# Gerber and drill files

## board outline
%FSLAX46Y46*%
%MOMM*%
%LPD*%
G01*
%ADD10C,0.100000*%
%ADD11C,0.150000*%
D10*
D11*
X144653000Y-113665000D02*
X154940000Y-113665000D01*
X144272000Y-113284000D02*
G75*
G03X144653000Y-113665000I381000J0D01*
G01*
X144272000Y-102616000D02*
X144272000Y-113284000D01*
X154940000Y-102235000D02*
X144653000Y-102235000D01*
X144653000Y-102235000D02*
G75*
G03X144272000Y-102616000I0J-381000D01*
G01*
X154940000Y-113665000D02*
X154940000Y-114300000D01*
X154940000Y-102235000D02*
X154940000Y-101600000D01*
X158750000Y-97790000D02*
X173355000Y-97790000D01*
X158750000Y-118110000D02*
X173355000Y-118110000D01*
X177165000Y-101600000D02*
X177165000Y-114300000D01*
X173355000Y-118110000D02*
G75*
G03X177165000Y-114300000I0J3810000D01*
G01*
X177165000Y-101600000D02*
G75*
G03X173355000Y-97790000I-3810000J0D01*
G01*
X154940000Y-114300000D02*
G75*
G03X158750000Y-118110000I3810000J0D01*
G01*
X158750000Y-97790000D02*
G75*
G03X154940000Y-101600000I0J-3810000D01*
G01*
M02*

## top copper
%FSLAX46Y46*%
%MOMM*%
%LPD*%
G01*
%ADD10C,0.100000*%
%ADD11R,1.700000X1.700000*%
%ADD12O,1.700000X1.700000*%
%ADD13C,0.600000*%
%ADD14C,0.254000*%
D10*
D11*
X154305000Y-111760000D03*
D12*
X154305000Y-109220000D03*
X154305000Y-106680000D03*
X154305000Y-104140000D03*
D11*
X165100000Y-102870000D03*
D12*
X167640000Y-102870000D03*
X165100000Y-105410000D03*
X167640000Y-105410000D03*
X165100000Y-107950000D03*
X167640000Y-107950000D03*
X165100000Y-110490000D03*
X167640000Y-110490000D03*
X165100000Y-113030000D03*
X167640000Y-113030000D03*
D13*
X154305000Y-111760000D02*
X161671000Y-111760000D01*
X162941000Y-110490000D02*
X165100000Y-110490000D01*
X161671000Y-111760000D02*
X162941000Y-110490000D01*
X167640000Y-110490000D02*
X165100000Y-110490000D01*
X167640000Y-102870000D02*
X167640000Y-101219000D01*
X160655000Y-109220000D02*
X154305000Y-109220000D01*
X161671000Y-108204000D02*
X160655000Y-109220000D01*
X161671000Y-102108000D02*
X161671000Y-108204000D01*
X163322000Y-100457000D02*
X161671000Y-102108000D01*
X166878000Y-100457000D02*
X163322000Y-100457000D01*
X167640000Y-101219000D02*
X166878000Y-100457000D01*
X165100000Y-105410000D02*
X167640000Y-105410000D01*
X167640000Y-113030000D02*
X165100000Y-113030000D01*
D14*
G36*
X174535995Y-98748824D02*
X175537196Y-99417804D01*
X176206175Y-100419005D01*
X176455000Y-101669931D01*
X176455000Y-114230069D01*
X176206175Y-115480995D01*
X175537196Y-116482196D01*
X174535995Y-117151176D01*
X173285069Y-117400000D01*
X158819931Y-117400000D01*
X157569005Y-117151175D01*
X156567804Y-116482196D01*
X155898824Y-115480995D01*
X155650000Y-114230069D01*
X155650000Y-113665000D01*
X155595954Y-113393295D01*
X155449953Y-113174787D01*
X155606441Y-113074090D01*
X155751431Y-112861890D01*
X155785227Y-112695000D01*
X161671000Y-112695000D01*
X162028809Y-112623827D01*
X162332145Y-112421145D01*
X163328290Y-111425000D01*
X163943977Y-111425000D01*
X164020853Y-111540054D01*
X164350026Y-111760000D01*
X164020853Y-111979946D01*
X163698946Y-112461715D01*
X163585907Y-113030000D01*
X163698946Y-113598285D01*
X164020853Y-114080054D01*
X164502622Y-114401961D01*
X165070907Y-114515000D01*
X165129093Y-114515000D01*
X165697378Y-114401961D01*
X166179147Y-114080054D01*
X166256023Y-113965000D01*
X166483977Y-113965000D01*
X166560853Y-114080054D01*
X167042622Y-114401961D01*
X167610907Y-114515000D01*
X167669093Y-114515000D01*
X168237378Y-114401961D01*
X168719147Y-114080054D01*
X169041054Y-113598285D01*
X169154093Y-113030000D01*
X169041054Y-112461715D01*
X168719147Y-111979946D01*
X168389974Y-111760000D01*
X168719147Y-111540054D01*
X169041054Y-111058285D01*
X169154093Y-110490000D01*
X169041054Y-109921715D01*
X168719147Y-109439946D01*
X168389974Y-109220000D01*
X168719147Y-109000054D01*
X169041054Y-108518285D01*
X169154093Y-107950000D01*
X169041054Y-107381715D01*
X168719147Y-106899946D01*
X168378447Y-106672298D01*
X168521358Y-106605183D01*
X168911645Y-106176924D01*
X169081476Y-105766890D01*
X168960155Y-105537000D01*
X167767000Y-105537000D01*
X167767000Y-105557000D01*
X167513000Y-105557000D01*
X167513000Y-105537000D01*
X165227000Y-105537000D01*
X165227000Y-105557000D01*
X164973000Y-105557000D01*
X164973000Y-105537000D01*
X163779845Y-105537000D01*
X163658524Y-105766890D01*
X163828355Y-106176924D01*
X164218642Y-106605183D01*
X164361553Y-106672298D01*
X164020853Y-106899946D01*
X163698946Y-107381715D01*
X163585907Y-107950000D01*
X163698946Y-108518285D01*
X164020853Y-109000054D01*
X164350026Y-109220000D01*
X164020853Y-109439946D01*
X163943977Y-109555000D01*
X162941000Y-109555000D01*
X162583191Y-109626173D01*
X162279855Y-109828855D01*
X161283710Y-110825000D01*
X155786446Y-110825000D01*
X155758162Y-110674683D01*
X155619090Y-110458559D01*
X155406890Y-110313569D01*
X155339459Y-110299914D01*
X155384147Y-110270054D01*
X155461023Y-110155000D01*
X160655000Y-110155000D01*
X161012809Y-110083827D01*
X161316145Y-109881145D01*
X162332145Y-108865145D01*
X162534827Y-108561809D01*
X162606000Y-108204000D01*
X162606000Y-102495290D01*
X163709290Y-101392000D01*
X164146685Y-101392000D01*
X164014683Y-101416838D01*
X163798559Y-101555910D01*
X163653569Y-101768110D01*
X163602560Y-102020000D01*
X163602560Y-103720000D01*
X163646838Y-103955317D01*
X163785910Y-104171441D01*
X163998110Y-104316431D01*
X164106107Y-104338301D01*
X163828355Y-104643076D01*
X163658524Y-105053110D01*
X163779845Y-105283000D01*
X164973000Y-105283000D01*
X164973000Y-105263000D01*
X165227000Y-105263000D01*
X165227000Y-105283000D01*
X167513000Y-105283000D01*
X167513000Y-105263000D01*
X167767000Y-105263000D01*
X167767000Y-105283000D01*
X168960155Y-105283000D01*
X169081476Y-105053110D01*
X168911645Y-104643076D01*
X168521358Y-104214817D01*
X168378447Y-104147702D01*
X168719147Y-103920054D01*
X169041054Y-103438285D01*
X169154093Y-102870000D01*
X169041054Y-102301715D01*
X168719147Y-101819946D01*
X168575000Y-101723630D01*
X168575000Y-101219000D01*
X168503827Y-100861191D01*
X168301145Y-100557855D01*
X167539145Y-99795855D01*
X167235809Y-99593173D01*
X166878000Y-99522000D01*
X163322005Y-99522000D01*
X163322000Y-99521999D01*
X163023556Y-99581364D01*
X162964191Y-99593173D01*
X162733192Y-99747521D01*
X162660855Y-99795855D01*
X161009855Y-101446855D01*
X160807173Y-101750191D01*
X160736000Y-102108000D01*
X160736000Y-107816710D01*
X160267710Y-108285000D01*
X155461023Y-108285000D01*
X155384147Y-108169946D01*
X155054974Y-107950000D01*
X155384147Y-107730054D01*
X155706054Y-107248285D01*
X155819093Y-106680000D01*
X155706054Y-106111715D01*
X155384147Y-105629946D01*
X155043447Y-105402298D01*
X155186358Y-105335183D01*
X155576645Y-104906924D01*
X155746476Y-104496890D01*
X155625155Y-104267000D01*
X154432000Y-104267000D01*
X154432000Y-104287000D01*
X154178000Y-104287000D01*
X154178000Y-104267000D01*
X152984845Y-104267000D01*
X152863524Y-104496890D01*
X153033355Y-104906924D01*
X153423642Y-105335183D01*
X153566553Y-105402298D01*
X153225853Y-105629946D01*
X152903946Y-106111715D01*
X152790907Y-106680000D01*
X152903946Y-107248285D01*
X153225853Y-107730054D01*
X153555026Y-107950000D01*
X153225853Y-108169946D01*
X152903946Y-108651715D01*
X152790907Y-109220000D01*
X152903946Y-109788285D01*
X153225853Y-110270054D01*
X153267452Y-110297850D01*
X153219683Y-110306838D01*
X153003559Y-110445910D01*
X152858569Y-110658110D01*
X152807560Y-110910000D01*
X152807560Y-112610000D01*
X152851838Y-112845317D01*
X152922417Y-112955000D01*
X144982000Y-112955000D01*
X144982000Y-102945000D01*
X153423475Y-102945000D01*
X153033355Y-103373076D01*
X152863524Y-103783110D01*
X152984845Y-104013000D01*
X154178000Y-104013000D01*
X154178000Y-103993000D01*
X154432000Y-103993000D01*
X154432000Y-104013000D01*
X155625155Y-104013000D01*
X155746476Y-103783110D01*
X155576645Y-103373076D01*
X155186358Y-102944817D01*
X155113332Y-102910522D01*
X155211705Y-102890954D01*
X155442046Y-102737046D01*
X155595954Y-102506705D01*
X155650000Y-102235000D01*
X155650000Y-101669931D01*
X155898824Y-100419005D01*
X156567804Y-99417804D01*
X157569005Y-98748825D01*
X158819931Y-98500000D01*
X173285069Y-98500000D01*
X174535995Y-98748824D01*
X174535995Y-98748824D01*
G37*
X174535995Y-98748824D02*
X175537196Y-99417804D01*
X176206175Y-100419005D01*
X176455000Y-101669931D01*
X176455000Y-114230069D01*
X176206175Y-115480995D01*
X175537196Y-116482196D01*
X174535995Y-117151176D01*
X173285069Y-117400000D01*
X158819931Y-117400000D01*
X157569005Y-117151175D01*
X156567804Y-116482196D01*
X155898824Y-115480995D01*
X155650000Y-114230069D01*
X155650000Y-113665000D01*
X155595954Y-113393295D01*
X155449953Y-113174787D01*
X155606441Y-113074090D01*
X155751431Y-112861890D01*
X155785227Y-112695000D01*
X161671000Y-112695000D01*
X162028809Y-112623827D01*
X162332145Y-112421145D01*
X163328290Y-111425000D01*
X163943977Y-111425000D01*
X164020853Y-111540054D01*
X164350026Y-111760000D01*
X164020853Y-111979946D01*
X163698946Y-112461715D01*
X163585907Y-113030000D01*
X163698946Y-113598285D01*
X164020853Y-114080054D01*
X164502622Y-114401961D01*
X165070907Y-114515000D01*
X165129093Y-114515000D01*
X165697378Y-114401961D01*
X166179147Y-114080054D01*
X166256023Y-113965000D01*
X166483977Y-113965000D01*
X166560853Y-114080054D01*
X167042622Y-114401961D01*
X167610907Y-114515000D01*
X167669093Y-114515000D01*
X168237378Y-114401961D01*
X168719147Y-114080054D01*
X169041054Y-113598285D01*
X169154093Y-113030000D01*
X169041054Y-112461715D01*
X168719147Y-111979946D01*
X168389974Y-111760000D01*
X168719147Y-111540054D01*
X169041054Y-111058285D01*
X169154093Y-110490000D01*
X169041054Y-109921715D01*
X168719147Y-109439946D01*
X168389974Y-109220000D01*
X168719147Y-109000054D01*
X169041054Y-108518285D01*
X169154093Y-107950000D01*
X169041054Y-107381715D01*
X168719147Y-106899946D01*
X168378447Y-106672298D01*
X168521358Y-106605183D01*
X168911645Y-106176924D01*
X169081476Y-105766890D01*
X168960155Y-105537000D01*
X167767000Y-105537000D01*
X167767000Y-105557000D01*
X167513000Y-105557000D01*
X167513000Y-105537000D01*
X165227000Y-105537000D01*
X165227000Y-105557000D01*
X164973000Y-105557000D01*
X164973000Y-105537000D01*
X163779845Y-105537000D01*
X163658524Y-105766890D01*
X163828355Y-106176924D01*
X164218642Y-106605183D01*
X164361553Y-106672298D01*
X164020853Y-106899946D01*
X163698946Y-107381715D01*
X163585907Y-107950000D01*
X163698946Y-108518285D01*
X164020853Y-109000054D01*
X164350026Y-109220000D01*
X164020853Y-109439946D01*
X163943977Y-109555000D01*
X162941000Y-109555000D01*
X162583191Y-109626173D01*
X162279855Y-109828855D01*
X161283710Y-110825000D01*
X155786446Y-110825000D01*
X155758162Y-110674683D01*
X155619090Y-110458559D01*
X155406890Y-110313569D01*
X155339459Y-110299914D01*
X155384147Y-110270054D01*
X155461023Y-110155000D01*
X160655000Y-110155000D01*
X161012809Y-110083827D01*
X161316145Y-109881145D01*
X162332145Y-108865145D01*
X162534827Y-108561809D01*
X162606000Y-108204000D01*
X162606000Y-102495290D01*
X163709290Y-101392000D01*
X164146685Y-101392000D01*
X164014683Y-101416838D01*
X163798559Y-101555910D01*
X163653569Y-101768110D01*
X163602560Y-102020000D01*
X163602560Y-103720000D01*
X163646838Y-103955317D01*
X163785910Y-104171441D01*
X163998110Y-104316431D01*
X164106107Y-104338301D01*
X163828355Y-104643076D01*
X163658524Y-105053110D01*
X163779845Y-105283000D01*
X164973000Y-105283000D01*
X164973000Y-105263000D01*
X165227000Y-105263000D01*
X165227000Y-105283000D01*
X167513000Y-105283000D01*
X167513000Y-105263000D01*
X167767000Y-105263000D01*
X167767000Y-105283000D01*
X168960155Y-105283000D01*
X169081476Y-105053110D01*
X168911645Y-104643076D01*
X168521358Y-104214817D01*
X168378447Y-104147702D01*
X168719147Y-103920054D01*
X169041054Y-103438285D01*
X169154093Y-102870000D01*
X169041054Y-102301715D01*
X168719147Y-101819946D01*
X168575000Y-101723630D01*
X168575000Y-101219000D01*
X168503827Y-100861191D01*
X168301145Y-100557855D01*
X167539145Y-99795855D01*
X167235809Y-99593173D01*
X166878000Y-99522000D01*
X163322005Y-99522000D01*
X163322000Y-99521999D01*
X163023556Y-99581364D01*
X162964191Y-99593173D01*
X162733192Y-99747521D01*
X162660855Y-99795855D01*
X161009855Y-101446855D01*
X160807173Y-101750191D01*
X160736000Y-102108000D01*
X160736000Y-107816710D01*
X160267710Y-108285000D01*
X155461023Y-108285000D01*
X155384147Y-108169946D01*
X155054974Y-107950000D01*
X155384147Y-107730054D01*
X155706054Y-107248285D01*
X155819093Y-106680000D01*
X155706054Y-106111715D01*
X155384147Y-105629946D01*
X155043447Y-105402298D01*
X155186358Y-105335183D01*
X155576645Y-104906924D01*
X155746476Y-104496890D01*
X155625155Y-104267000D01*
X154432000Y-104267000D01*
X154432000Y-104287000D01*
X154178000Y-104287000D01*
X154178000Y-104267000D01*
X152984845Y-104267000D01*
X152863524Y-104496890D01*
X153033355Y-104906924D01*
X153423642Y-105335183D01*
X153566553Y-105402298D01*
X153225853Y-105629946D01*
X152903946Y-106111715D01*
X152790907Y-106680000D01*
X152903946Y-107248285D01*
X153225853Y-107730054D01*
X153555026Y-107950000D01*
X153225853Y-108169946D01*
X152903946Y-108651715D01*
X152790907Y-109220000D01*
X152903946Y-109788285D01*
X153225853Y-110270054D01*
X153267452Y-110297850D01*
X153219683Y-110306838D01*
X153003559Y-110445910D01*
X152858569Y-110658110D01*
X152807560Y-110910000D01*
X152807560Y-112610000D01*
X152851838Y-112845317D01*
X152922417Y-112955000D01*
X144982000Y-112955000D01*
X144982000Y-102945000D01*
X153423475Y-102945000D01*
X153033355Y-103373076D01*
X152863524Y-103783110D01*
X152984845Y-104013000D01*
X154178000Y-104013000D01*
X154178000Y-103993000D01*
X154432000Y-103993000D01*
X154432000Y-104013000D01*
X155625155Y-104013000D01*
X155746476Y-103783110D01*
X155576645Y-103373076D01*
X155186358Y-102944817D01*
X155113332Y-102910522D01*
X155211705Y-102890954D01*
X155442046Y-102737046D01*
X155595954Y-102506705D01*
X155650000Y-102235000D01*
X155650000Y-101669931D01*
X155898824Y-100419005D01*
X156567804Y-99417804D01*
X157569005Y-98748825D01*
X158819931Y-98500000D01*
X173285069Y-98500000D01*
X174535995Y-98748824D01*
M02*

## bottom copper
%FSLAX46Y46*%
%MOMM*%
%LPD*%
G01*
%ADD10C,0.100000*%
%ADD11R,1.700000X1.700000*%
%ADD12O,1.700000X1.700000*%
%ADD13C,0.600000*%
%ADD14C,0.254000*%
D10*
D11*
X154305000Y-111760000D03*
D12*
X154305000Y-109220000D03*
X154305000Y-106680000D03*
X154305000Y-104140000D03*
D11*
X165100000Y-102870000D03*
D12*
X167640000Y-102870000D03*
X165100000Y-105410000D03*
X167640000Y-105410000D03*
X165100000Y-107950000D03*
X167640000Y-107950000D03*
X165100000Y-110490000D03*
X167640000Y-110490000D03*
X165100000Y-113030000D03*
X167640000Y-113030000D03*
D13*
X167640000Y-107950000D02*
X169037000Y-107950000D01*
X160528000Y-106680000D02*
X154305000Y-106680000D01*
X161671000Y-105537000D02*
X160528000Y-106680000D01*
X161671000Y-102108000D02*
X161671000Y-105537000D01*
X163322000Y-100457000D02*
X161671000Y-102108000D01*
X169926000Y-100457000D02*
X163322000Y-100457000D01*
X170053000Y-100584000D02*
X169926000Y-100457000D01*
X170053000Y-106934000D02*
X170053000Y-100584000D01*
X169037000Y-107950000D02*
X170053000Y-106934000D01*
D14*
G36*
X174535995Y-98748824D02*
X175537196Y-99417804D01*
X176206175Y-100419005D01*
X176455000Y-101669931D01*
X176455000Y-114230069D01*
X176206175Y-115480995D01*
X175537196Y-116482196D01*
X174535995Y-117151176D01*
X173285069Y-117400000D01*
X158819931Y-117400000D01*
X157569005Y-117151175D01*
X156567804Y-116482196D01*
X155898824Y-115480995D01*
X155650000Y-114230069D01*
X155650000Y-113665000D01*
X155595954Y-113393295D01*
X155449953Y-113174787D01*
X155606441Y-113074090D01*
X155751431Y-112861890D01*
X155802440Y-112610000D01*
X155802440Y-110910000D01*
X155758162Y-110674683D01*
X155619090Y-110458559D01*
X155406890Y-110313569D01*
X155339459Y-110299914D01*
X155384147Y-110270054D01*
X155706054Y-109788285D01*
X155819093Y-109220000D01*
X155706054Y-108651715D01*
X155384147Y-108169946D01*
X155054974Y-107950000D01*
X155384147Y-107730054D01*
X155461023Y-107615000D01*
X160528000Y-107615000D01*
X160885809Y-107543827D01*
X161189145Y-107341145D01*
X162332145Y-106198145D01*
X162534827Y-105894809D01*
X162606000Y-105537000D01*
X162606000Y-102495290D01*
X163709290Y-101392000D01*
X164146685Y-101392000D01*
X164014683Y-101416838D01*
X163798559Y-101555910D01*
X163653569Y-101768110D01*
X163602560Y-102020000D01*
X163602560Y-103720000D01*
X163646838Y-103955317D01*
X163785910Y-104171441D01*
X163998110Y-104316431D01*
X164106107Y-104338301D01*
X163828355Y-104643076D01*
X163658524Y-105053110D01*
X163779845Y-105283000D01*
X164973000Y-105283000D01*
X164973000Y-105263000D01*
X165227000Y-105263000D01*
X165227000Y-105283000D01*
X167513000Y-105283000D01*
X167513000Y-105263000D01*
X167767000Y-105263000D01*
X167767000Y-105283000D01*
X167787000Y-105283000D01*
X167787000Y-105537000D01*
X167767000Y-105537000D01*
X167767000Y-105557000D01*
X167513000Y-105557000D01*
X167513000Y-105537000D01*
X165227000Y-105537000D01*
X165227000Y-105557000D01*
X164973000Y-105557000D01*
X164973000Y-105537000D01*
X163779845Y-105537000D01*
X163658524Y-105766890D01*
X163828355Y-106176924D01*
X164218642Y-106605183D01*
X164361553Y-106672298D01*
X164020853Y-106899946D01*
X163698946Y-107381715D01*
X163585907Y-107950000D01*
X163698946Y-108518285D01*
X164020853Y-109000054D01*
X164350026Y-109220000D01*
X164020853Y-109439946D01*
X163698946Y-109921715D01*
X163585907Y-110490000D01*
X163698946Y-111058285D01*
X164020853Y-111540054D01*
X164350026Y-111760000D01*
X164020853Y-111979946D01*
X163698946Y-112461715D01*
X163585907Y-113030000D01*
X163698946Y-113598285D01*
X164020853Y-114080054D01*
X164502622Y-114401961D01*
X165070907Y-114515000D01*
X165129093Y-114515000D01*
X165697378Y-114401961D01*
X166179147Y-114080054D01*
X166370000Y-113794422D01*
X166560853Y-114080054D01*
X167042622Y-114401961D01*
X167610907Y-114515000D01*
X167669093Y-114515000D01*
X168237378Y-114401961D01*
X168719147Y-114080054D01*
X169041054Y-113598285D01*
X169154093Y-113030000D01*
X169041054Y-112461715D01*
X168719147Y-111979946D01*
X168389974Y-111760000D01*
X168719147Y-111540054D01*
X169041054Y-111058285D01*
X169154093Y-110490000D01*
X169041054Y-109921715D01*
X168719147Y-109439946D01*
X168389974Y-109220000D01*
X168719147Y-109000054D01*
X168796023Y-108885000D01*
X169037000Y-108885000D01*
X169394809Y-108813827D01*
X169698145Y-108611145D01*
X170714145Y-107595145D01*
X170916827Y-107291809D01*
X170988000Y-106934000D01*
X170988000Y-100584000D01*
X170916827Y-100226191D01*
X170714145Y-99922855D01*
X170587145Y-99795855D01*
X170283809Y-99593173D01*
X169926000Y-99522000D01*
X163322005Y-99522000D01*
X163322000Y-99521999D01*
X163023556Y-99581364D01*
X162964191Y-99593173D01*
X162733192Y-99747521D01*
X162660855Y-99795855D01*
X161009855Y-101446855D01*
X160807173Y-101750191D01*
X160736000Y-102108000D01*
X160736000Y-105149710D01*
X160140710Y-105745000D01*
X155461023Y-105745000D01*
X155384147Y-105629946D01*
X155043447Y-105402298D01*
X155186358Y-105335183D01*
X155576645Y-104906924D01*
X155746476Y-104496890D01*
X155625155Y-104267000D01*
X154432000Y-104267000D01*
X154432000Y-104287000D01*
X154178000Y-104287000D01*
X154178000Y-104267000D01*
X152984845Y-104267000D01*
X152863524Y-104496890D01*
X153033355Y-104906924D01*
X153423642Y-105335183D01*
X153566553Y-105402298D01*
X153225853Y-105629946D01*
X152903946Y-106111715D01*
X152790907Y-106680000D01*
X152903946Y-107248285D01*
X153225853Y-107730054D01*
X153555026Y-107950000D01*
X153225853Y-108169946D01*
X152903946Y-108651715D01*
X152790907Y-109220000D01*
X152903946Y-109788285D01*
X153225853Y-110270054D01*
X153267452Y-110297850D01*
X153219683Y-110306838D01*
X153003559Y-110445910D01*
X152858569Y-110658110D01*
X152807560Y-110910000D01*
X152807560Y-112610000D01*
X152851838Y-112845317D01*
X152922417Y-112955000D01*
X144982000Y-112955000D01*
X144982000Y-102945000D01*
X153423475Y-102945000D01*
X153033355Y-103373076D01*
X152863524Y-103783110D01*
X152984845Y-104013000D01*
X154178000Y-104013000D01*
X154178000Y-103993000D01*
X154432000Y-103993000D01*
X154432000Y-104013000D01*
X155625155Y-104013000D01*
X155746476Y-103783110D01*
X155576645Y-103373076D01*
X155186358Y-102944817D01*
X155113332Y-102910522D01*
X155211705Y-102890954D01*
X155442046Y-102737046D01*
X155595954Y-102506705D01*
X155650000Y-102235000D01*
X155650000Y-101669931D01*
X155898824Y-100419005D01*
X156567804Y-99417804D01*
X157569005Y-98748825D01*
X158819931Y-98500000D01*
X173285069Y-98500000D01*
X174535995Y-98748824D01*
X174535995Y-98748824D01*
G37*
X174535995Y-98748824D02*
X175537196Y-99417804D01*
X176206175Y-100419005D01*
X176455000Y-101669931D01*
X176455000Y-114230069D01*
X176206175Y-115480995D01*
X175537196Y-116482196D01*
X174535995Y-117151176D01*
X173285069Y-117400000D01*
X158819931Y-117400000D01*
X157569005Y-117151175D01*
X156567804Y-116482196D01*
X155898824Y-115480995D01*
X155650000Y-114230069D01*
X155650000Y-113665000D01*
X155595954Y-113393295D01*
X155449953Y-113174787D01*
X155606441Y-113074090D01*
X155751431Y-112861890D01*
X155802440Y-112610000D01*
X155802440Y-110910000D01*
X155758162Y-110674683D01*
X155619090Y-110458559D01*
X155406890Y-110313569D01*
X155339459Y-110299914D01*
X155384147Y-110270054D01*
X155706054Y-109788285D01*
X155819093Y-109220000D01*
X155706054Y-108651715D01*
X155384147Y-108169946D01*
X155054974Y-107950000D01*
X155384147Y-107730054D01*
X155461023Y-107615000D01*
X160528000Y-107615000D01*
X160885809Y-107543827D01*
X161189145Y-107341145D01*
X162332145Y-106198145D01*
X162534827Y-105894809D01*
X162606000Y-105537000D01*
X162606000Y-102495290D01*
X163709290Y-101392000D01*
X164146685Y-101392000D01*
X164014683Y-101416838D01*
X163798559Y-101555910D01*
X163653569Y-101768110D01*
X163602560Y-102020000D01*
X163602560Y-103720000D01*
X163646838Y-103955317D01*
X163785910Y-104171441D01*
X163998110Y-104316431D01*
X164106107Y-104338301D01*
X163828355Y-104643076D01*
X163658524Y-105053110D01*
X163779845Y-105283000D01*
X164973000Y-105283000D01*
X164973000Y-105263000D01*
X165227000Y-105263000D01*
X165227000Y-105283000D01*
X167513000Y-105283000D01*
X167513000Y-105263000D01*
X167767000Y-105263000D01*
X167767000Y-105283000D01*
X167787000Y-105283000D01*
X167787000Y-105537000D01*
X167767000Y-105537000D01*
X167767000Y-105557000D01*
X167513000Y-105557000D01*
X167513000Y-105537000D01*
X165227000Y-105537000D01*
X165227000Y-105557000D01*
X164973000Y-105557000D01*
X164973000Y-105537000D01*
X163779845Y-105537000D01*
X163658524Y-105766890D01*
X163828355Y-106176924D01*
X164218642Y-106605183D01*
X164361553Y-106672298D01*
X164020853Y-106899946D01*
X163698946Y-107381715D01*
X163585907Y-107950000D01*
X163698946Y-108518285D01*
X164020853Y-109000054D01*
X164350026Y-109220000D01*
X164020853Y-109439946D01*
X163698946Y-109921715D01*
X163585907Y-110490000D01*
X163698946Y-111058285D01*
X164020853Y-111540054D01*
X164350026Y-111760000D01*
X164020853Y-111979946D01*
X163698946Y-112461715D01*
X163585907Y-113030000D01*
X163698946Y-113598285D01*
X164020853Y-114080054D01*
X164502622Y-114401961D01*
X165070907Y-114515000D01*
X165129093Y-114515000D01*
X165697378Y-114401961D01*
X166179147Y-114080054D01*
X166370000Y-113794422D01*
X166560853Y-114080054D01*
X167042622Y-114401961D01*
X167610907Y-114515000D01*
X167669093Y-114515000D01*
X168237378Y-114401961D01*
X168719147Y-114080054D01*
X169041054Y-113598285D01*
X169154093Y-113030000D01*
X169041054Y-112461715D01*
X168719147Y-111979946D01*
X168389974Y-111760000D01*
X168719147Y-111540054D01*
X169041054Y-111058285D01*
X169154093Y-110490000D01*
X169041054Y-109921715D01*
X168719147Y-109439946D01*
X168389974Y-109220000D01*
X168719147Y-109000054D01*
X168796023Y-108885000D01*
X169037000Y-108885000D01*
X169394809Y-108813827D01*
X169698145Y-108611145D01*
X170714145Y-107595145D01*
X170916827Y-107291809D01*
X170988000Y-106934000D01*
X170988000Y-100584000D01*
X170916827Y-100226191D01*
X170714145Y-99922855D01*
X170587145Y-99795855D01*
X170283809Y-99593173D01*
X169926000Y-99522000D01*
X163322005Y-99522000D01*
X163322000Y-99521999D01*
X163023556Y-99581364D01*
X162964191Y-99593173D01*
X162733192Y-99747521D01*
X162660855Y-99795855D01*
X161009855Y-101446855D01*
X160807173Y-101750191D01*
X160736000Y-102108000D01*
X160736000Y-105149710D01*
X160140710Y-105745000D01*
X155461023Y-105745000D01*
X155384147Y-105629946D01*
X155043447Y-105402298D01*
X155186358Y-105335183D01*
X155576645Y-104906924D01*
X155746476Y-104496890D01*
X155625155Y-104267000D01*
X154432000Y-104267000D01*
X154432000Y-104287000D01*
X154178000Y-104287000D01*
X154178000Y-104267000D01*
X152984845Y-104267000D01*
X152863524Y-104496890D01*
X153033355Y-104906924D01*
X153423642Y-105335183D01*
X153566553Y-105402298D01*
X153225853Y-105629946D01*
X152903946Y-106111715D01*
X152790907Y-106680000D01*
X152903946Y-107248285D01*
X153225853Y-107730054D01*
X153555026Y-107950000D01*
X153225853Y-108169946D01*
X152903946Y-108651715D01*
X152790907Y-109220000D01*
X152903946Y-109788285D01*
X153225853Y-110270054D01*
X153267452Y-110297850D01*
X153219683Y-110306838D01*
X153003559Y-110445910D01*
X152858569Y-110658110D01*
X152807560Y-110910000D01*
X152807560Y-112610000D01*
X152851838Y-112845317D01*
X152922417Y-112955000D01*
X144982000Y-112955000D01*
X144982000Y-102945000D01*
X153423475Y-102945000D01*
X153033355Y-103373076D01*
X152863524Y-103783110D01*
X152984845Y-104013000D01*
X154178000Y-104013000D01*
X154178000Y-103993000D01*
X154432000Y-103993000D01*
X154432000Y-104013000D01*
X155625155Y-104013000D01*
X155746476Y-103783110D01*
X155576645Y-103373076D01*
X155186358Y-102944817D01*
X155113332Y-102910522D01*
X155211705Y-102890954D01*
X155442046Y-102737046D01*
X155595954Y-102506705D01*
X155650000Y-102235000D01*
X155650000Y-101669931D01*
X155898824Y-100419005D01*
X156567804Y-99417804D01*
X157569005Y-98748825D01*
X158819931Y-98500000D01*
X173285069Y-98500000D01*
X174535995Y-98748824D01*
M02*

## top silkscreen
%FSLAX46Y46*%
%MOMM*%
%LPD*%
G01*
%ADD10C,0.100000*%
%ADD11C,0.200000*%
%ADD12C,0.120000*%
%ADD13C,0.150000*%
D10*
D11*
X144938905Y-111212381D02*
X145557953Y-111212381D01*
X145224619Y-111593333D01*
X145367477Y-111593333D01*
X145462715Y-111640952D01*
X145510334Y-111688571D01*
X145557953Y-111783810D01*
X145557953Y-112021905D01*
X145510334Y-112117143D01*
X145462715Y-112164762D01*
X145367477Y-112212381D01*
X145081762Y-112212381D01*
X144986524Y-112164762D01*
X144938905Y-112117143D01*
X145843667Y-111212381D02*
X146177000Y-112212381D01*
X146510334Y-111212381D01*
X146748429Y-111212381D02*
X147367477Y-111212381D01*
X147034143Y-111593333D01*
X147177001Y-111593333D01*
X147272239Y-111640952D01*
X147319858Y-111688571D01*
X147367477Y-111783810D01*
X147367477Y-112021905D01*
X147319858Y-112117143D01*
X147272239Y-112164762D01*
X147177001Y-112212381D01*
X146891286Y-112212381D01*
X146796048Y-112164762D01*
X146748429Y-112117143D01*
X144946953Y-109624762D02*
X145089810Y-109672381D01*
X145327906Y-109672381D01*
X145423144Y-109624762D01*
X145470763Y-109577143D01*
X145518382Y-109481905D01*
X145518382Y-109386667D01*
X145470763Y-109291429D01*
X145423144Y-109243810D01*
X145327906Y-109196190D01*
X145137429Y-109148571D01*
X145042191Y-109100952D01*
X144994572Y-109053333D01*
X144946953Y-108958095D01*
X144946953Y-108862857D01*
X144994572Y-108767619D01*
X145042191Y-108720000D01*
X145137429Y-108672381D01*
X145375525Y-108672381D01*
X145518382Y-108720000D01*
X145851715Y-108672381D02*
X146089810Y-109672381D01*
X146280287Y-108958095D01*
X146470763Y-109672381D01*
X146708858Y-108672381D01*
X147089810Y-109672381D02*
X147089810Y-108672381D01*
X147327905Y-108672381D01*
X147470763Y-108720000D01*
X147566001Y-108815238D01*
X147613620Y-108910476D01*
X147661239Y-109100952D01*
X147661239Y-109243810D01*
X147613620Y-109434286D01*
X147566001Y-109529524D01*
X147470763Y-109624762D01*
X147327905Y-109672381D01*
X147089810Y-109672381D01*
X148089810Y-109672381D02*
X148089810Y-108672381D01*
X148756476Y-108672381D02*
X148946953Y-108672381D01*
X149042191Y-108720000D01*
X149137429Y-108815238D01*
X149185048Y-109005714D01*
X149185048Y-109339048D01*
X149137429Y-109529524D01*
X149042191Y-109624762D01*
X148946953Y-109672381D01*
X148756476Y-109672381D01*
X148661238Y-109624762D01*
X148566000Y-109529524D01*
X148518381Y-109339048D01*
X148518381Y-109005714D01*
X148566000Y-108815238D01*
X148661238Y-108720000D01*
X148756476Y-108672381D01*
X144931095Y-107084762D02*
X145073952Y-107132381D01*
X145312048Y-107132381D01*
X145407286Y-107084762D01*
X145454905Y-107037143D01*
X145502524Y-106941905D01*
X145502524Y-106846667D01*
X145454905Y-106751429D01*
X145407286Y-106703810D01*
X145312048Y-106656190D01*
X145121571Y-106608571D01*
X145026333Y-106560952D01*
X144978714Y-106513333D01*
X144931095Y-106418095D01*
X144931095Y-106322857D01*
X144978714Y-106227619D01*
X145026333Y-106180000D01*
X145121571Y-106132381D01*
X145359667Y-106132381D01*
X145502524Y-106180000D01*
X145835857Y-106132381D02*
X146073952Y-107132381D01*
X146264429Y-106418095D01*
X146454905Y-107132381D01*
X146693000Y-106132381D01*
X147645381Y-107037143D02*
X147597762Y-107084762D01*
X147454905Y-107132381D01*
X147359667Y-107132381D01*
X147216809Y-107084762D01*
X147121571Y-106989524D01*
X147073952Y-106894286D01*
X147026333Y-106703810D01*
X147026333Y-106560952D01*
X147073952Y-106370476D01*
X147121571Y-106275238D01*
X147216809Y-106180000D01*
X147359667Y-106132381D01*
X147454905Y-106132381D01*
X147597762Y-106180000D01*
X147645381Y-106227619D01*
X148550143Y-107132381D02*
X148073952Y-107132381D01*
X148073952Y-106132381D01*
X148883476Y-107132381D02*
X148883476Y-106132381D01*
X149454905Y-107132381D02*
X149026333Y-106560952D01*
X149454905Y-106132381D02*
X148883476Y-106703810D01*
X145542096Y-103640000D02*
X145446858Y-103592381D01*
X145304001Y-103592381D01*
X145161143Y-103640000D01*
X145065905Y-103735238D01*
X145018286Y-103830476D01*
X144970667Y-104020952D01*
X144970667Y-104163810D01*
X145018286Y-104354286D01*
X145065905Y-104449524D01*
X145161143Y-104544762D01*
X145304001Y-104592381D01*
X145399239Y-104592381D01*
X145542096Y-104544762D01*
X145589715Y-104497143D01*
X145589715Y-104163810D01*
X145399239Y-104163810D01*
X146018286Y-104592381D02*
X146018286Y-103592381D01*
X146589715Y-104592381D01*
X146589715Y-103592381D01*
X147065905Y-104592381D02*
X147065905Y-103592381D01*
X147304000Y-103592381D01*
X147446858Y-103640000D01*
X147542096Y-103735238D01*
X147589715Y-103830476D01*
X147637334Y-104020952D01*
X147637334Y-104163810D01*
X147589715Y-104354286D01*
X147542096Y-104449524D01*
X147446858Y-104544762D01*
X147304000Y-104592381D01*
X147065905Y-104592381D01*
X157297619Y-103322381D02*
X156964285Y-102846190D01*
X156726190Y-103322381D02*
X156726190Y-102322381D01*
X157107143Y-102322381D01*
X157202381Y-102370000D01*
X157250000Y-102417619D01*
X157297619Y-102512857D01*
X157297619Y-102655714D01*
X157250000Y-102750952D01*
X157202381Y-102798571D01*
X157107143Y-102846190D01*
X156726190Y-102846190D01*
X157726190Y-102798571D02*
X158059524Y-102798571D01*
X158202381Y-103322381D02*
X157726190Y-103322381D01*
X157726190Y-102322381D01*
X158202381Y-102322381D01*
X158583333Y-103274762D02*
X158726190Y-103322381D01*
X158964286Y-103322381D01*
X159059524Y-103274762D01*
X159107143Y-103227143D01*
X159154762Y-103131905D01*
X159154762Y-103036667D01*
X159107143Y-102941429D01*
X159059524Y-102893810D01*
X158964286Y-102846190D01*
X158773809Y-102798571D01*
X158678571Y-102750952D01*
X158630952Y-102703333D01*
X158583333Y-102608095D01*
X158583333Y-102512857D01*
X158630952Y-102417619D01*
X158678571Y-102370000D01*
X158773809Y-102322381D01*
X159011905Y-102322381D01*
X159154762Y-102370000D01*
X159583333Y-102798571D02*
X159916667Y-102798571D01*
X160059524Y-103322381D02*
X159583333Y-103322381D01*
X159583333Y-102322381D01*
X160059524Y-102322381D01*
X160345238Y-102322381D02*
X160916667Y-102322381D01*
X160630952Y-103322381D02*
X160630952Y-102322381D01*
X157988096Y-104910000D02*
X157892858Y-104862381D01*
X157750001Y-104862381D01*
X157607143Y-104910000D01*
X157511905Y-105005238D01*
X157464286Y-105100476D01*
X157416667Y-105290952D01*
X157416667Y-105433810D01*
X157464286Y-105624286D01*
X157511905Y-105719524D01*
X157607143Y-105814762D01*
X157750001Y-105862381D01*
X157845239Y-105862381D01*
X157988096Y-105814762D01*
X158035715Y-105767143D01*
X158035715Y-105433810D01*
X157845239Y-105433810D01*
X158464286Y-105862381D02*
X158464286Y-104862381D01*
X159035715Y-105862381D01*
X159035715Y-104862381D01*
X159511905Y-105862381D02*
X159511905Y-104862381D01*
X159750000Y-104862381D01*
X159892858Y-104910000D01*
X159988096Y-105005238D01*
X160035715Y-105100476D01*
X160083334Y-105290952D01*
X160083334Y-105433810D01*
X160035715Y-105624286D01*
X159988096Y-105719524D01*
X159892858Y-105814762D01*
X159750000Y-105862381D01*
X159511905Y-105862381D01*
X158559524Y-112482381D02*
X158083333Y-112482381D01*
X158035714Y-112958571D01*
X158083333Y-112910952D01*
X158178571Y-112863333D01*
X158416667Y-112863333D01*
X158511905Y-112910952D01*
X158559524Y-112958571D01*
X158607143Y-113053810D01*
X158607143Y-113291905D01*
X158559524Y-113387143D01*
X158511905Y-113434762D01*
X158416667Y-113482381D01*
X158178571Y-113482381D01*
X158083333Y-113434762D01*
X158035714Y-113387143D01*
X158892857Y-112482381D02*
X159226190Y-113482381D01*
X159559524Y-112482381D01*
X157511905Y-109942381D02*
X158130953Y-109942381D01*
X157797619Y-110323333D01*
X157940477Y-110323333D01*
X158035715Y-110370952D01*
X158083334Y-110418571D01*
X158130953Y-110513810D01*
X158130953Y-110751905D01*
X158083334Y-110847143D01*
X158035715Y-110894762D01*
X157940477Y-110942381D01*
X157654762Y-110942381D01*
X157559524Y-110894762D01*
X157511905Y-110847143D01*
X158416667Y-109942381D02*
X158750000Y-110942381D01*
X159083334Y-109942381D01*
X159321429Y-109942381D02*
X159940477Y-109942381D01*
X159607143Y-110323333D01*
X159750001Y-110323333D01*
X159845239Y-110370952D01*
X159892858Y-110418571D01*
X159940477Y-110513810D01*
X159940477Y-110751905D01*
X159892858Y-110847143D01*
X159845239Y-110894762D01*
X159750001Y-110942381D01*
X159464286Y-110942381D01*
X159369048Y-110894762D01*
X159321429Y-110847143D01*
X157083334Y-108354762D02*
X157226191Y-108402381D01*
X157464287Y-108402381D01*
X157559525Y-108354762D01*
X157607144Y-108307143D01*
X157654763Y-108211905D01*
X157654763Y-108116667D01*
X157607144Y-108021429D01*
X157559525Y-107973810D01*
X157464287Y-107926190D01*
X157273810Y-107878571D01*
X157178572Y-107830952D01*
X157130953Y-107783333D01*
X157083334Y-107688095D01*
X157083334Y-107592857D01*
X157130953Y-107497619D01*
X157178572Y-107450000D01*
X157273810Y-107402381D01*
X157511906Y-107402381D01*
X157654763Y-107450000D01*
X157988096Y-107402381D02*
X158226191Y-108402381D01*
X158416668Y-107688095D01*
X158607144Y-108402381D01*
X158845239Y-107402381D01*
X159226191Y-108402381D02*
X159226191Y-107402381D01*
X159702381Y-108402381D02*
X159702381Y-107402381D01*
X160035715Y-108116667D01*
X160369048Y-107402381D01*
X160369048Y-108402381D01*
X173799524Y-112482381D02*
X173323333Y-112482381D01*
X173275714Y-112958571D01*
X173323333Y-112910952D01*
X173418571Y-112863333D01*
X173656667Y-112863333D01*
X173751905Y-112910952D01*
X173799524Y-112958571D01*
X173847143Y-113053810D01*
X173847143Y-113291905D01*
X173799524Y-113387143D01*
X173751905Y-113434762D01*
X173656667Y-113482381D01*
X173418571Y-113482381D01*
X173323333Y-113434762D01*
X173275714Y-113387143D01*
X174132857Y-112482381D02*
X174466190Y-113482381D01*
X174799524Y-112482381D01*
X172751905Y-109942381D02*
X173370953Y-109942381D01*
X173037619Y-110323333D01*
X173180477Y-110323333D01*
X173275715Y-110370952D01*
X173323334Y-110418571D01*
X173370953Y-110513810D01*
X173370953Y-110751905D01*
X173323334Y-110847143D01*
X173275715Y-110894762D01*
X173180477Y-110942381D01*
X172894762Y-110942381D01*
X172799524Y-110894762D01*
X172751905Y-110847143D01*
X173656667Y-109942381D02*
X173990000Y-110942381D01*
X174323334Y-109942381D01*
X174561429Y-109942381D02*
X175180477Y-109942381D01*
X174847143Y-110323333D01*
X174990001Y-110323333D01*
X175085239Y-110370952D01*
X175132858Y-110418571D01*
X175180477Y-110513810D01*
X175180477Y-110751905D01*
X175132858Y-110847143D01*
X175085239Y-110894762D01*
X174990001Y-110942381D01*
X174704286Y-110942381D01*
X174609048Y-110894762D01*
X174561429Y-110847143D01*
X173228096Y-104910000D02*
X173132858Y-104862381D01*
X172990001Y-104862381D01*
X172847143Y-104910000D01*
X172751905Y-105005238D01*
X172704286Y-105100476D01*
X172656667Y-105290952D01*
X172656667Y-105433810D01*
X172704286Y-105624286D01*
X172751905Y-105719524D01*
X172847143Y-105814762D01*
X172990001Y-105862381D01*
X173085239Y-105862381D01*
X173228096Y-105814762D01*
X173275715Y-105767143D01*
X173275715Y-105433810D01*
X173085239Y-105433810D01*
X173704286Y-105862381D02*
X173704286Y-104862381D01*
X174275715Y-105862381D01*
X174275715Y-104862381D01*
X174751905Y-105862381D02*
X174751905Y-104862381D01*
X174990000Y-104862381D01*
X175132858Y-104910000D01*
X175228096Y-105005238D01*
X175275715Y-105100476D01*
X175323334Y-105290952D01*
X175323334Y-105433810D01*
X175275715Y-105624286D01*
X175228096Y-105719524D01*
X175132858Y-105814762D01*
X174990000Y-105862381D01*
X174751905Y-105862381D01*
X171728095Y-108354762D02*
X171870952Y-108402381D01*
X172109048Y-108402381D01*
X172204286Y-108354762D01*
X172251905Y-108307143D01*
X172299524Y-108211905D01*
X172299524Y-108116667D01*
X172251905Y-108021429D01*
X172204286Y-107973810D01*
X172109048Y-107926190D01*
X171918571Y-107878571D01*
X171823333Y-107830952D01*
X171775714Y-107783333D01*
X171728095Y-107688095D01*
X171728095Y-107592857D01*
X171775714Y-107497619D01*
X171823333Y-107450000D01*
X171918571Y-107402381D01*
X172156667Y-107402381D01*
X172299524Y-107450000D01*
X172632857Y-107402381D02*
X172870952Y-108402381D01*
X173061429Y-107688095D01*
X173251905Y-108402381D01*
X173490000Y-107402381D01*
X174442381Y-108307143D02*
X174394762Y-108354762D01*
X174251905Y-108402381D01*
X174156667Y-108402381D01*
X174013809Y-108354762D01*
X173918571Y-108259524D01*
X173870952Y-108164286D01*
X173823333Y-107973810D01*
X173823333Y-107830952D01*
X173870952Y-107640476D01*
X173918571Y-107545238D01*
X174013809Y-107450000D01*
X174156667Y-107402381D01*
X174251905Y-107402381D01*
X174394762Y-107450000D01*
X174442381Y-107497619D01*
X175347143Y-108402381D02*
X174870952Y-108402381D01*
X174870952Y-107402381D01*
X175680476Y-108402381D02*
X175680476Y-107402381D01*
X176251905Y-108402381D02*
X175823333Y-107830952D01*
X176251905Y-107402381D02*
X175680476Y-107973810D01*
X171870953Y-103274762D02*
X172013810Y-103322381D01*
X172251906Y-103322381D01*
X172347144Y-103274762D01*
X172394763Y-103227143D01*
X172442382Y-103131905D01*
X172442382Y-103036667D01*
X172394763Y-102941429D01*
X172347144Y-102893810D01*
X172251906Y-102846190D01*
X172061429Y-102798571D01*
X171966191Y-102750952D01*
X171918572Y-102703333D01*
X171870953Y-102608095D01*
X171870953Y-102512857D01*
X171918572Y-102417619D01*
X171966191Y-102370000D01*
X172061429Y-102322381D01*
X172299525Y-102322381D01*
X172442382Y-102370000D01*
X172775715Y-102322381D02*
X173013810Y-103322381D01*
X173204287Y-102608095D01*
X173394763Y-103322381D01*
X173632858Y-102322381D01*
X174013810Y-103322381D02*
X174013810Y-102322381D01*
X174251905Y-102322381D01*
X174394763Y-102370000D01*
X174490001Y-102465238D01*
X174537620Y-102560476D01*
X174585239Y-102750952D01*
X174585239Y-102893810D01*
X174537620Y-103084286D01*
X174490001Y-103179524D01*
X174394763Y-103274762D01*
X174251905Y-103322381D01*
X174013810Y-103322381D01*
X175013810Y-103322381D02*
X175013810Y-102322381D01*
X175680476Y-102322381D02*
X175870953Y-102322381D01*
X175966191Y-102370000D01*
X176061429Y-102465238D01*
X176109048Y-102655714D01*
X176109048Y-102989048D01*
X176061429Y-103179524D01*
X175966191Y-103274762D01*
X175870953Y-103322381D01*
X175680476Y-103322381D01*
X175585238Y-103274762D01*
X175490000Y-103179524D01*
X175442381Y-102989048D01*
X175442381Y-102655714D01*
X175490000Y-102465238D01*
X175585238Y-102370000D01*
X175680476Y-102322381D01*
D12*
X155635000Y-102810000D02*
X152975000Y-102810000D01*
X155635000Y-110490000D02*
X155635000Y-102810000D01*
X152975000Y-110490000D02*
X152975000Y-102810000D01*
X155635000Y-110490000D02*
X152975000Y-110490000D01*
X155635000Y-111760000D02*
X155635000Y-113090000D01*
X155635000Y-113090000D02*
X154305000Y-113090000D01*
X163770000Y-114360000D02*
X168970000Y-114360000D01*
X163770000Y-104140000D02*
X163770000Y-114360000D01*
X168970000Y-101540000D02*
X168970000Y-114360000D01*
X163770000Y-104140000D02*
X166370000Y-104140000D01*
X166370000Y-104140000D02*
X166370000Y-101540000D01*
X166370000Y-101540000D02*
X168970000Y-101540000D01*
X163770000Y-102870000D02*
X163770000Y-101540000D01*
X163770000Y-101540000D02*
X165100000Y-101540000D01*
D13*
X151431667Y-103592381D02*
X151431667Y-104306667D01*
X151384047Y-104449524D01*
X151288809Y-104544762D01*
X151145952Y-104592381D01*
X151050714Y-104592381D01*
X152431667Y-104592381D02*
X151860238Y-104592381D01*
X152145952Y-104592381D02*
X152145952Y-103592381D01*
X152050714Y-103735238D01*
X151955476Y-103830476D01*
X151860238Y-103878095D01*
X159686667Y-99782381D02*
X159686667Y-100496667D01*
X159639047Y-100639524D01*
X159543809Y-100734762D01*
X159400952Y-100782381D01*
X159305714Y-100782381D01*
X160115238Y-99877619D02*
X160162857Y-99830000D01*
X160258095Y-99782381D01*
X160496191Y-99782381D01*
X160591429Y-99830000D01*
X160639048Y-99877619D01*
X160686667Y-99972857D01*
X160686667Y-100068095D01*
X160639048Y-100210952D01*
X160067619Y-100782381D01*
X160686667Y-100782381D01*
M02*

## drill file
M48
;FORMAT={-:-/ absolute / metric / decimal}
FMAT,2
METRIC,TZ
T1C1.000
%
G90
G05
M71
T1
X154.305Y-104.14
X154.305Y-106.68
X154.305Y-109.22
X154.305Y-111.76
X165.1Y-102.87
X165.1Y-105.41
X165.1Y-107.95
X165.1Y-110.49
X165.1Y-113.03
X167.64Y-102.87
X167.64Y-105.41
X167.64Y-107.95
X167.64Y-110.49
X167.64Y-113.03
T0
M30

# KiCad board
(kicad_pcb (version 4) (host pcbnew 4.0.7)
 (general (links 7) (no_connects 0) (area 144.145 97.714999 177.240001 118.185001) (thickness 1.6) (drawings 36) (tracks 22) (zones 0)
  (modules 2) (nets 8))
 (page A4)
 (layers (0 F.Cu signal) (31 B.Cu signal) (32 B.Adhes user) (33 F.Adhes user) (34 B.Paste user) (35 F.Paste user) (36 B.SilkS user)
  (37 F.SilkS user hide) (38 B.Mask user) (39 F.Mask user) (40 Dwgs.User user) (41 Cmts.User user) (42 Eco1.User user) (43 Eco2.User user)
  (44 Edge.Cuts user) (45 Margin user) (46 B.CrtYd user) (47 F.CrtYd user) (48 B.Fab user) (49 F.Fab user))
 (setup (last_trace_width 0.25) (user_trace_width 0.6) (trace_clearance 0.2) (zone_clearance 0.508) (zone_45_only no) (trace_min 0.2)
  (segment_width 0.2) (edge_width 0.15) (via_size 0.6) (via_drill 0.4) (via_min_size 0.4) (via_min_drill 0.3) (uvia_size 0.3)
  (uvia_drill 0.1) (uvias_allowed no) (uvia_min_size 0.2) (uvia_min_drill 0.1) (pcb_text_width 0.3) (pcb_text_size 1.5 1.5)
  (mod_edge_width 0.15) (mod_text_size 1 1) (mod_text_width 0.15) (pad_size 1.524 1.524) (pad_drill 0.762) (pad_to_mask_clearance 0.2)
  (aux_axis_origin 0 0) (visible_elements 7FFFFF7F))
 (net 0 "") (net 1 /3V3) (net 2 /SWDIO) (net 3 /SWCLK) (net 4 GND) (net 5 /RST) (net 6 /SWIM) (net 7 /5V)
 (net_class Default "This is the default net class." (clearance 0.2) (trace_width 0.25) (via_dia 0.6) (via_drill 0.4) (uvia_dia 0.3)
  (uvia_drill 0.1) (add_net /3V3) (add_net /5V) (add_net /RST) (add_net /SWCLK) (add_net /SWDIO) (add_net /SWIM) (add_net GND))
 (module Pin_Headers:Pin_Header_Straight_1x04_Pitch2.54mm (layer F.Cu) (at 154.305 111.76 180)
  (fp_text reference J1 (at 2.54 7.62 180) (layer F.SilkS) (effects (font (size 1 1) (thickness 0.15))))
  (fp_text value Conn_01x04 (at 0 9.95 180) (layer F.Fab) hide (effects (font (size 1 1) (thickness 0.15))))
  (fp_line (start -1.33 8.95) (end 1.33 8.95) (layer F.SilkS) (width 0.12))
  (fp_line (start -1.33 1.27) (end -1.33 8.95) (layer F.SilkS) (width 0.12))
  (fp_line (start 1.33 1.27) (end 1.33 8.95) (layer F.SilkS) (width 0.12))
  (fp_line (start -1.33 1.27) (end 1.33 1.27) (layer F.SilkS) (width 0.12))
  (fp_line (start -1.33 0) (end -1.33 -1.33) (layer F.SilkS) (width 0.12))
  (fp_line (start -1.33 -1.33) (end 0 -1.33) (layer F.SilkS) (width 0.12))
  (pad 1 thru_hole rect (at 0 0 180) (size 1.7 1.7) (drill 1) (layers *.Cu *.Mask) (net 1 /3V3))
  (pad 2 thru_hole oval (at 0 2.54 180) (size 1.7 1.7) (drill 1) (layers *.Cu *.Mask) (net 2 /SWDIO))
  (pad 3 thru_hole oval (at 0 5.08 180) (size 1.7 1.7) (drill 1) (layers *.Cu *.Mask) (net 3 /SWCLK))
  (pad 4 thru_hole oval (at 0 7.62 180) (size 1.7 1.7) (drill 1) (layers *.Cu *.Mask) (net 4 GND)))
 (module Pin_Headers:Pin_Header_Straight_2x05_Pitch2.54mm (layer F.Cu) (at 165.1 102.87)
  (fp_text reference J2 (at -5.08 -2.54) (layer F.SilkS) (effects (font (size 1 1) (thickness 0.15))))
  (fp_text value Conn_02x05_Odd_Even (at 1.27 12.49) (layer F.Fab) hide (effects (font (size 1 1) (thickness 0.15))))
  (fp_line (start -1.33 11.49) (end 3.87 11.49) (layer F.SilkS) (width 0.12))
  (fp_line (start -1.33 1.27) (end -1.33 11.49) (layer F.SilkS) (width 0.12))
  (fp_line (start 3.87 -1.33) (end 3.87 11.49) (layer F.SilkS) (width 0.12))
  (fp_line (start -1.33 1.27) (end 1.27 1.27) (layer F.SilkS) (width 0.12))
  (fp_line (start 1.27 1.27) (end 1.27 -1.33) (layer F.SilkS) (width 0.12))
  (fp_line (start 1.27 -1.33) (end 3.87 -1.33) (layer F.SilkS) (width 0.12))
  (fp_line (start -1.33 0) (end -1.33 -1.33) (layer F.SilkS) (width 0.12))
  (fp_line (start -1.33 -1.33) (end 0 -1.33) (layer F.SilkS) (width 0.12))
  (pad 1 thru_hole rect (at 0 0) (size 1.7 1.7) (drill 1) (layers *.Cu *.Mask) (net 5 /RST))
  (pad 2 thru_hole oval (at 2.54 0) (size 1.7 1.7) (drill 1) (layers *.Cu *.Mask) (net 2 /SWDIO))
  (pad 3 thru_hole oval (at 0 2.54) (size 1.7 1.7) (drill 1) (layers *.Cu *.Mask) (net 4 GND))
  (pad 4 thru_hole oval (at 2.54 2.54) (size 1.7 1.7) (drill 1) (layers *.Cu *.Mask) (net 4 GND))
  (pad 5 thru_hole oval (at 0 5.08) (size 1.7 1.7) (drill 1) (layers *.Cu *.Mask) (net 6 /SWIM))
  (pad 6 thru_hole oval (at 2.54 5.08) (size 1.7 1.7) (drill 1) (layers *.Cu *.Mask) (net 3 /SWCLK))
  (pad 7 thru_hole oval (at 0 7.62) (size 1.7 1.7) (drill 1) (layers *.Cu *.Mask) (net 1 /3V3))
  (pad 8 thru_hole oval (at 2.54 7.62) (size 1.7 1.7) (drill 1) (layers *.Cu *.Mask) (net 1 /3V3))
  (pad 9 thru_hole oval (at 0 10.16) (size 1.7 1.7) (drill 1) (layers *.Cu *.Mask) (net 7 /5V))
  (pad 10 thru_hole oval (at 2.54 10.16) (size 1.7 1.7) (drill 1) (layers *.Cu *.Mask) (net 7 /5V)))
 (gr_line (start 144.653 113.665) (end 154.94 113.665) (angle 90) (layer Edge.Cuts) (width 0.15))
 (gr_arc (start 144.653 113.284) (end 144.653 113.665) (angle 90) (layer Edge.Cuts) (width 0.15))
 (gr_line (start 144.272 102.616) (end 144.272 113.284) (angle 90) (layer Edge.Cuts) (width 0.15))
 (gr_line (start 154.94 102.235) (end 144.653 102.235) (angle 90) (layer Edge.Cuts) (width 0.15))
 (gr_arc (start 144.653 102.616) (end 144.272 102.616) (angle 90) (layer Edge.Cuts) (width 0.15))
 (gr_line (start 154.94 113.665) (end 154.94 114.3) (angle 90) (layer Edge.Cuts) (width 0.15))
 (gr_line (start 154.94 102.235) (end 154.94 101.6) (angle 90) (layer Edge.Cuts) (width 0.15))
 (gr_line (start 158.75 97.79) (end 173.355 97.79) (angle 90) (layer Edge.Cuts) (width 0.15))
 (gr_line (start 158.75 118.11) (end 173.355 118.11) (angle 90) (layer Edge.Cuts) (width 0.15))
 (gr_line (start 177.165 101.6) (end 177.165 114.3) (angle 90) (layer Edge.Cuts) (width 0.15))
 (gr_arc (start 173.355 114.3) (end 177.165 114.3) (angle 90) (layer Edge.Cuts) (width 0.15))
 (gr_arc (start 173.355 101.6) (end 173.355 97.79) (angle 90) (layer Edge.Cuts) (width 0.15))
 (gr_arc (start 158.75 114.3) (end 158.75 118.11) (angle 90) (layer Edge.Cuts) (width 0.15))
 (gr_arc (start 158.75 101.6) (end 154.94 101.6) (angle 90) (layer Edge.Cuts) (width 0.15))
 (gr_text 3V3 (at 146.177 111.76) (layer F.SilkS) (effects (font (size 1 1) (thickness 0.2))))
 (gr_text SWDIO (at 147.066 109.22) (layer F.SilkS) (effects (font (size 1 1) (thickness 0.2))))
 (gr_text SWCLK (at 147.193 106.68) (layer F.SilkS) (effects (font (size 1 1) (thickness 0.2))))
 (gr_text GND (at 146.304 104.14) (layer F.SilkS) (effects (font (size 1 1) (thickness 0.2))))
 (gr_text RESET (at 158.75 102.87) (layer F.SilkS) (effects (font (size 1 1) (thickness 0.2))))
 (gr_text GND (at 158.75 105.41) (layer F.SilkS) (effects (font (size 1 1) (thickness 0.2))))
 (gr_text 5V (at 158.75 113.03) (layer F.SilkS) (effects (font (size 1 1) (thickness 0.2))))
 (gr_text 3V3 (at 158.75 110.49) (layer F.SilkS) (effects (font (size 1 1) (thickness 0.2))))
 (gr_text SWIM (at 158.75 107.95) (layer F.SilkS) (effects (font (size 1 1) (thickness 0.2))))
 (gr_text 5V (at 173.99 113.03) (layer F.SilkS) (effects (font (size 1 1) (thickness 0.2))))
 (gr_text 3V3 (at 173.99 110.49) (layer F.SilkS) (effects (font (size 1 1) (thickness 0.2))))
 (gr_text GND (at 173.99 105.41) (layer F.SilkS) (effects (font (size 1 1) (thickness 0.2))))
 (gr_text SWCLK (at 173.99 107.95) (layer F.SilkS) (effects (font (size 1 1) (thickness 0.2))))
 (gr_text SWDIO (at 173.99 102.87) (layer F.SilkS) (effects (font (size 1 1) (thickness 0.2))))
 (segment (start 154.305 111.76) (end 161.671 111.76) (width 0.6) (layer F.Cu) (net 1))
 (segment (start 162.941 110.49) (end 165.1 110.49) (width 0.6) (layer F.Cu) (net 1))
 (segment (start 161.671 111.76) (end 162.941 110.49) (width 0.6) (layer F.Cu) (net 1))
 (segment (start 167.64 110.49) (end 165.1 110.49) (width 0.6) (layer F.Cu) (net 1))
 (segment (start 167.64 102.87) (end 167.64 101.219) (width 0.6) (layer F.Cu) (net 2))
 (segment (start 160.655 109.22) (end 154.305 109.22) (width 0.6) (layer F.Cu) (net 2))
 (segment (start 161.671 108.204) (end 160.655 109.22) (width 0.6) (layer F.Cu) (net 2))
 (segment (start 161.671 102.108) (end 161.671 108.204) (width 0.6) (layer F.Cu) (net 2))
 (segment (start 163.322 100.457) (end 161.671 102.108) (width 0.6) (layer F.Cu) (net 2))
 (segment (start 166.878 100.457) (end 163.322 100.457) (width 0.6) (layer F.Cu) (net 2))
 (segment (start 167.64 101.219) (end 166.878 100.457) (width 0.6) (layer F.Cu) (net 2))
 (segment (start 167.64 107.95) (end 169.037 107.95) (width 0.6) (layer B.Cu) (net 3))
 (segment (start 160.528 106.68) (end 154.305 106.68) (width 0.6) (layer B.Cu) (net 3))
 (segment (start 161.671 105.537) (end 160.528 106.68) (width 0.6) (layer B.Cu) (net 3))
 (segment (start 161.671 102.108) (end 161.671 105.537) (width 0.6) (layer B.Cu) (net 3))
 (segment (start 163.322 100.457) (end 161.671 102.108) (width 0.6) (layer B.Cu) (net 3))
 (segment (start 169.926 100.457) (end 163.322 100.457) (width 0.6) (layer B.Cu) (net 3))
 (segment (start 170.053 100.584) (end 169.926 100.457) (width 0.6) (layer B.Cu) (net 3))
 (segment (start 170.053 106.934) (end 170.053 100.584) (width 0.6) (layer B.Cu) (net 3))
 (segment (start 169.037 107.95) (end 170.053 106.934) (width 0.6) (layer B.Cu) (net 3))
 (segment (start 165.1 105.41) (end 167.64 105.41) (width 0.6) (layer F.Cu) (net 4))
 (segment (start 167.64 113.03) (end 165.1 113.03) (width 0.6) (layer F.Cu) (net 7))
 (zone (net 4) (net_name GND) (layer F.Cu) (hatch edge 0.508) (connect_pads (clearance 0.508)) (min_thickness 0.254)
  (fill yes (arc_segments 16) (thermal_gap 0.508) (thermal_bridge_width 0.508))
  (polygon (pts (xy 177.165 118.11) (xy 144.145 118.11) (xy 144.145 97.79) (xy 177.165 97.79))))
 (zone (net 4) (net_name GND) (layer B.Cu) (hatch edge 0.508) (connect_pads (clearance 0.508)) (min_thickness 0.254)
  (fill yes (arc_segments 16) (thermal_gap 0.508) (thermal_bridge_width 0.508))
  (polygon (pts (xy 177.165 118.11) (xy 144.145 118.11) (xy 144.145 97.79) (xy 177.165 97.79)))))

